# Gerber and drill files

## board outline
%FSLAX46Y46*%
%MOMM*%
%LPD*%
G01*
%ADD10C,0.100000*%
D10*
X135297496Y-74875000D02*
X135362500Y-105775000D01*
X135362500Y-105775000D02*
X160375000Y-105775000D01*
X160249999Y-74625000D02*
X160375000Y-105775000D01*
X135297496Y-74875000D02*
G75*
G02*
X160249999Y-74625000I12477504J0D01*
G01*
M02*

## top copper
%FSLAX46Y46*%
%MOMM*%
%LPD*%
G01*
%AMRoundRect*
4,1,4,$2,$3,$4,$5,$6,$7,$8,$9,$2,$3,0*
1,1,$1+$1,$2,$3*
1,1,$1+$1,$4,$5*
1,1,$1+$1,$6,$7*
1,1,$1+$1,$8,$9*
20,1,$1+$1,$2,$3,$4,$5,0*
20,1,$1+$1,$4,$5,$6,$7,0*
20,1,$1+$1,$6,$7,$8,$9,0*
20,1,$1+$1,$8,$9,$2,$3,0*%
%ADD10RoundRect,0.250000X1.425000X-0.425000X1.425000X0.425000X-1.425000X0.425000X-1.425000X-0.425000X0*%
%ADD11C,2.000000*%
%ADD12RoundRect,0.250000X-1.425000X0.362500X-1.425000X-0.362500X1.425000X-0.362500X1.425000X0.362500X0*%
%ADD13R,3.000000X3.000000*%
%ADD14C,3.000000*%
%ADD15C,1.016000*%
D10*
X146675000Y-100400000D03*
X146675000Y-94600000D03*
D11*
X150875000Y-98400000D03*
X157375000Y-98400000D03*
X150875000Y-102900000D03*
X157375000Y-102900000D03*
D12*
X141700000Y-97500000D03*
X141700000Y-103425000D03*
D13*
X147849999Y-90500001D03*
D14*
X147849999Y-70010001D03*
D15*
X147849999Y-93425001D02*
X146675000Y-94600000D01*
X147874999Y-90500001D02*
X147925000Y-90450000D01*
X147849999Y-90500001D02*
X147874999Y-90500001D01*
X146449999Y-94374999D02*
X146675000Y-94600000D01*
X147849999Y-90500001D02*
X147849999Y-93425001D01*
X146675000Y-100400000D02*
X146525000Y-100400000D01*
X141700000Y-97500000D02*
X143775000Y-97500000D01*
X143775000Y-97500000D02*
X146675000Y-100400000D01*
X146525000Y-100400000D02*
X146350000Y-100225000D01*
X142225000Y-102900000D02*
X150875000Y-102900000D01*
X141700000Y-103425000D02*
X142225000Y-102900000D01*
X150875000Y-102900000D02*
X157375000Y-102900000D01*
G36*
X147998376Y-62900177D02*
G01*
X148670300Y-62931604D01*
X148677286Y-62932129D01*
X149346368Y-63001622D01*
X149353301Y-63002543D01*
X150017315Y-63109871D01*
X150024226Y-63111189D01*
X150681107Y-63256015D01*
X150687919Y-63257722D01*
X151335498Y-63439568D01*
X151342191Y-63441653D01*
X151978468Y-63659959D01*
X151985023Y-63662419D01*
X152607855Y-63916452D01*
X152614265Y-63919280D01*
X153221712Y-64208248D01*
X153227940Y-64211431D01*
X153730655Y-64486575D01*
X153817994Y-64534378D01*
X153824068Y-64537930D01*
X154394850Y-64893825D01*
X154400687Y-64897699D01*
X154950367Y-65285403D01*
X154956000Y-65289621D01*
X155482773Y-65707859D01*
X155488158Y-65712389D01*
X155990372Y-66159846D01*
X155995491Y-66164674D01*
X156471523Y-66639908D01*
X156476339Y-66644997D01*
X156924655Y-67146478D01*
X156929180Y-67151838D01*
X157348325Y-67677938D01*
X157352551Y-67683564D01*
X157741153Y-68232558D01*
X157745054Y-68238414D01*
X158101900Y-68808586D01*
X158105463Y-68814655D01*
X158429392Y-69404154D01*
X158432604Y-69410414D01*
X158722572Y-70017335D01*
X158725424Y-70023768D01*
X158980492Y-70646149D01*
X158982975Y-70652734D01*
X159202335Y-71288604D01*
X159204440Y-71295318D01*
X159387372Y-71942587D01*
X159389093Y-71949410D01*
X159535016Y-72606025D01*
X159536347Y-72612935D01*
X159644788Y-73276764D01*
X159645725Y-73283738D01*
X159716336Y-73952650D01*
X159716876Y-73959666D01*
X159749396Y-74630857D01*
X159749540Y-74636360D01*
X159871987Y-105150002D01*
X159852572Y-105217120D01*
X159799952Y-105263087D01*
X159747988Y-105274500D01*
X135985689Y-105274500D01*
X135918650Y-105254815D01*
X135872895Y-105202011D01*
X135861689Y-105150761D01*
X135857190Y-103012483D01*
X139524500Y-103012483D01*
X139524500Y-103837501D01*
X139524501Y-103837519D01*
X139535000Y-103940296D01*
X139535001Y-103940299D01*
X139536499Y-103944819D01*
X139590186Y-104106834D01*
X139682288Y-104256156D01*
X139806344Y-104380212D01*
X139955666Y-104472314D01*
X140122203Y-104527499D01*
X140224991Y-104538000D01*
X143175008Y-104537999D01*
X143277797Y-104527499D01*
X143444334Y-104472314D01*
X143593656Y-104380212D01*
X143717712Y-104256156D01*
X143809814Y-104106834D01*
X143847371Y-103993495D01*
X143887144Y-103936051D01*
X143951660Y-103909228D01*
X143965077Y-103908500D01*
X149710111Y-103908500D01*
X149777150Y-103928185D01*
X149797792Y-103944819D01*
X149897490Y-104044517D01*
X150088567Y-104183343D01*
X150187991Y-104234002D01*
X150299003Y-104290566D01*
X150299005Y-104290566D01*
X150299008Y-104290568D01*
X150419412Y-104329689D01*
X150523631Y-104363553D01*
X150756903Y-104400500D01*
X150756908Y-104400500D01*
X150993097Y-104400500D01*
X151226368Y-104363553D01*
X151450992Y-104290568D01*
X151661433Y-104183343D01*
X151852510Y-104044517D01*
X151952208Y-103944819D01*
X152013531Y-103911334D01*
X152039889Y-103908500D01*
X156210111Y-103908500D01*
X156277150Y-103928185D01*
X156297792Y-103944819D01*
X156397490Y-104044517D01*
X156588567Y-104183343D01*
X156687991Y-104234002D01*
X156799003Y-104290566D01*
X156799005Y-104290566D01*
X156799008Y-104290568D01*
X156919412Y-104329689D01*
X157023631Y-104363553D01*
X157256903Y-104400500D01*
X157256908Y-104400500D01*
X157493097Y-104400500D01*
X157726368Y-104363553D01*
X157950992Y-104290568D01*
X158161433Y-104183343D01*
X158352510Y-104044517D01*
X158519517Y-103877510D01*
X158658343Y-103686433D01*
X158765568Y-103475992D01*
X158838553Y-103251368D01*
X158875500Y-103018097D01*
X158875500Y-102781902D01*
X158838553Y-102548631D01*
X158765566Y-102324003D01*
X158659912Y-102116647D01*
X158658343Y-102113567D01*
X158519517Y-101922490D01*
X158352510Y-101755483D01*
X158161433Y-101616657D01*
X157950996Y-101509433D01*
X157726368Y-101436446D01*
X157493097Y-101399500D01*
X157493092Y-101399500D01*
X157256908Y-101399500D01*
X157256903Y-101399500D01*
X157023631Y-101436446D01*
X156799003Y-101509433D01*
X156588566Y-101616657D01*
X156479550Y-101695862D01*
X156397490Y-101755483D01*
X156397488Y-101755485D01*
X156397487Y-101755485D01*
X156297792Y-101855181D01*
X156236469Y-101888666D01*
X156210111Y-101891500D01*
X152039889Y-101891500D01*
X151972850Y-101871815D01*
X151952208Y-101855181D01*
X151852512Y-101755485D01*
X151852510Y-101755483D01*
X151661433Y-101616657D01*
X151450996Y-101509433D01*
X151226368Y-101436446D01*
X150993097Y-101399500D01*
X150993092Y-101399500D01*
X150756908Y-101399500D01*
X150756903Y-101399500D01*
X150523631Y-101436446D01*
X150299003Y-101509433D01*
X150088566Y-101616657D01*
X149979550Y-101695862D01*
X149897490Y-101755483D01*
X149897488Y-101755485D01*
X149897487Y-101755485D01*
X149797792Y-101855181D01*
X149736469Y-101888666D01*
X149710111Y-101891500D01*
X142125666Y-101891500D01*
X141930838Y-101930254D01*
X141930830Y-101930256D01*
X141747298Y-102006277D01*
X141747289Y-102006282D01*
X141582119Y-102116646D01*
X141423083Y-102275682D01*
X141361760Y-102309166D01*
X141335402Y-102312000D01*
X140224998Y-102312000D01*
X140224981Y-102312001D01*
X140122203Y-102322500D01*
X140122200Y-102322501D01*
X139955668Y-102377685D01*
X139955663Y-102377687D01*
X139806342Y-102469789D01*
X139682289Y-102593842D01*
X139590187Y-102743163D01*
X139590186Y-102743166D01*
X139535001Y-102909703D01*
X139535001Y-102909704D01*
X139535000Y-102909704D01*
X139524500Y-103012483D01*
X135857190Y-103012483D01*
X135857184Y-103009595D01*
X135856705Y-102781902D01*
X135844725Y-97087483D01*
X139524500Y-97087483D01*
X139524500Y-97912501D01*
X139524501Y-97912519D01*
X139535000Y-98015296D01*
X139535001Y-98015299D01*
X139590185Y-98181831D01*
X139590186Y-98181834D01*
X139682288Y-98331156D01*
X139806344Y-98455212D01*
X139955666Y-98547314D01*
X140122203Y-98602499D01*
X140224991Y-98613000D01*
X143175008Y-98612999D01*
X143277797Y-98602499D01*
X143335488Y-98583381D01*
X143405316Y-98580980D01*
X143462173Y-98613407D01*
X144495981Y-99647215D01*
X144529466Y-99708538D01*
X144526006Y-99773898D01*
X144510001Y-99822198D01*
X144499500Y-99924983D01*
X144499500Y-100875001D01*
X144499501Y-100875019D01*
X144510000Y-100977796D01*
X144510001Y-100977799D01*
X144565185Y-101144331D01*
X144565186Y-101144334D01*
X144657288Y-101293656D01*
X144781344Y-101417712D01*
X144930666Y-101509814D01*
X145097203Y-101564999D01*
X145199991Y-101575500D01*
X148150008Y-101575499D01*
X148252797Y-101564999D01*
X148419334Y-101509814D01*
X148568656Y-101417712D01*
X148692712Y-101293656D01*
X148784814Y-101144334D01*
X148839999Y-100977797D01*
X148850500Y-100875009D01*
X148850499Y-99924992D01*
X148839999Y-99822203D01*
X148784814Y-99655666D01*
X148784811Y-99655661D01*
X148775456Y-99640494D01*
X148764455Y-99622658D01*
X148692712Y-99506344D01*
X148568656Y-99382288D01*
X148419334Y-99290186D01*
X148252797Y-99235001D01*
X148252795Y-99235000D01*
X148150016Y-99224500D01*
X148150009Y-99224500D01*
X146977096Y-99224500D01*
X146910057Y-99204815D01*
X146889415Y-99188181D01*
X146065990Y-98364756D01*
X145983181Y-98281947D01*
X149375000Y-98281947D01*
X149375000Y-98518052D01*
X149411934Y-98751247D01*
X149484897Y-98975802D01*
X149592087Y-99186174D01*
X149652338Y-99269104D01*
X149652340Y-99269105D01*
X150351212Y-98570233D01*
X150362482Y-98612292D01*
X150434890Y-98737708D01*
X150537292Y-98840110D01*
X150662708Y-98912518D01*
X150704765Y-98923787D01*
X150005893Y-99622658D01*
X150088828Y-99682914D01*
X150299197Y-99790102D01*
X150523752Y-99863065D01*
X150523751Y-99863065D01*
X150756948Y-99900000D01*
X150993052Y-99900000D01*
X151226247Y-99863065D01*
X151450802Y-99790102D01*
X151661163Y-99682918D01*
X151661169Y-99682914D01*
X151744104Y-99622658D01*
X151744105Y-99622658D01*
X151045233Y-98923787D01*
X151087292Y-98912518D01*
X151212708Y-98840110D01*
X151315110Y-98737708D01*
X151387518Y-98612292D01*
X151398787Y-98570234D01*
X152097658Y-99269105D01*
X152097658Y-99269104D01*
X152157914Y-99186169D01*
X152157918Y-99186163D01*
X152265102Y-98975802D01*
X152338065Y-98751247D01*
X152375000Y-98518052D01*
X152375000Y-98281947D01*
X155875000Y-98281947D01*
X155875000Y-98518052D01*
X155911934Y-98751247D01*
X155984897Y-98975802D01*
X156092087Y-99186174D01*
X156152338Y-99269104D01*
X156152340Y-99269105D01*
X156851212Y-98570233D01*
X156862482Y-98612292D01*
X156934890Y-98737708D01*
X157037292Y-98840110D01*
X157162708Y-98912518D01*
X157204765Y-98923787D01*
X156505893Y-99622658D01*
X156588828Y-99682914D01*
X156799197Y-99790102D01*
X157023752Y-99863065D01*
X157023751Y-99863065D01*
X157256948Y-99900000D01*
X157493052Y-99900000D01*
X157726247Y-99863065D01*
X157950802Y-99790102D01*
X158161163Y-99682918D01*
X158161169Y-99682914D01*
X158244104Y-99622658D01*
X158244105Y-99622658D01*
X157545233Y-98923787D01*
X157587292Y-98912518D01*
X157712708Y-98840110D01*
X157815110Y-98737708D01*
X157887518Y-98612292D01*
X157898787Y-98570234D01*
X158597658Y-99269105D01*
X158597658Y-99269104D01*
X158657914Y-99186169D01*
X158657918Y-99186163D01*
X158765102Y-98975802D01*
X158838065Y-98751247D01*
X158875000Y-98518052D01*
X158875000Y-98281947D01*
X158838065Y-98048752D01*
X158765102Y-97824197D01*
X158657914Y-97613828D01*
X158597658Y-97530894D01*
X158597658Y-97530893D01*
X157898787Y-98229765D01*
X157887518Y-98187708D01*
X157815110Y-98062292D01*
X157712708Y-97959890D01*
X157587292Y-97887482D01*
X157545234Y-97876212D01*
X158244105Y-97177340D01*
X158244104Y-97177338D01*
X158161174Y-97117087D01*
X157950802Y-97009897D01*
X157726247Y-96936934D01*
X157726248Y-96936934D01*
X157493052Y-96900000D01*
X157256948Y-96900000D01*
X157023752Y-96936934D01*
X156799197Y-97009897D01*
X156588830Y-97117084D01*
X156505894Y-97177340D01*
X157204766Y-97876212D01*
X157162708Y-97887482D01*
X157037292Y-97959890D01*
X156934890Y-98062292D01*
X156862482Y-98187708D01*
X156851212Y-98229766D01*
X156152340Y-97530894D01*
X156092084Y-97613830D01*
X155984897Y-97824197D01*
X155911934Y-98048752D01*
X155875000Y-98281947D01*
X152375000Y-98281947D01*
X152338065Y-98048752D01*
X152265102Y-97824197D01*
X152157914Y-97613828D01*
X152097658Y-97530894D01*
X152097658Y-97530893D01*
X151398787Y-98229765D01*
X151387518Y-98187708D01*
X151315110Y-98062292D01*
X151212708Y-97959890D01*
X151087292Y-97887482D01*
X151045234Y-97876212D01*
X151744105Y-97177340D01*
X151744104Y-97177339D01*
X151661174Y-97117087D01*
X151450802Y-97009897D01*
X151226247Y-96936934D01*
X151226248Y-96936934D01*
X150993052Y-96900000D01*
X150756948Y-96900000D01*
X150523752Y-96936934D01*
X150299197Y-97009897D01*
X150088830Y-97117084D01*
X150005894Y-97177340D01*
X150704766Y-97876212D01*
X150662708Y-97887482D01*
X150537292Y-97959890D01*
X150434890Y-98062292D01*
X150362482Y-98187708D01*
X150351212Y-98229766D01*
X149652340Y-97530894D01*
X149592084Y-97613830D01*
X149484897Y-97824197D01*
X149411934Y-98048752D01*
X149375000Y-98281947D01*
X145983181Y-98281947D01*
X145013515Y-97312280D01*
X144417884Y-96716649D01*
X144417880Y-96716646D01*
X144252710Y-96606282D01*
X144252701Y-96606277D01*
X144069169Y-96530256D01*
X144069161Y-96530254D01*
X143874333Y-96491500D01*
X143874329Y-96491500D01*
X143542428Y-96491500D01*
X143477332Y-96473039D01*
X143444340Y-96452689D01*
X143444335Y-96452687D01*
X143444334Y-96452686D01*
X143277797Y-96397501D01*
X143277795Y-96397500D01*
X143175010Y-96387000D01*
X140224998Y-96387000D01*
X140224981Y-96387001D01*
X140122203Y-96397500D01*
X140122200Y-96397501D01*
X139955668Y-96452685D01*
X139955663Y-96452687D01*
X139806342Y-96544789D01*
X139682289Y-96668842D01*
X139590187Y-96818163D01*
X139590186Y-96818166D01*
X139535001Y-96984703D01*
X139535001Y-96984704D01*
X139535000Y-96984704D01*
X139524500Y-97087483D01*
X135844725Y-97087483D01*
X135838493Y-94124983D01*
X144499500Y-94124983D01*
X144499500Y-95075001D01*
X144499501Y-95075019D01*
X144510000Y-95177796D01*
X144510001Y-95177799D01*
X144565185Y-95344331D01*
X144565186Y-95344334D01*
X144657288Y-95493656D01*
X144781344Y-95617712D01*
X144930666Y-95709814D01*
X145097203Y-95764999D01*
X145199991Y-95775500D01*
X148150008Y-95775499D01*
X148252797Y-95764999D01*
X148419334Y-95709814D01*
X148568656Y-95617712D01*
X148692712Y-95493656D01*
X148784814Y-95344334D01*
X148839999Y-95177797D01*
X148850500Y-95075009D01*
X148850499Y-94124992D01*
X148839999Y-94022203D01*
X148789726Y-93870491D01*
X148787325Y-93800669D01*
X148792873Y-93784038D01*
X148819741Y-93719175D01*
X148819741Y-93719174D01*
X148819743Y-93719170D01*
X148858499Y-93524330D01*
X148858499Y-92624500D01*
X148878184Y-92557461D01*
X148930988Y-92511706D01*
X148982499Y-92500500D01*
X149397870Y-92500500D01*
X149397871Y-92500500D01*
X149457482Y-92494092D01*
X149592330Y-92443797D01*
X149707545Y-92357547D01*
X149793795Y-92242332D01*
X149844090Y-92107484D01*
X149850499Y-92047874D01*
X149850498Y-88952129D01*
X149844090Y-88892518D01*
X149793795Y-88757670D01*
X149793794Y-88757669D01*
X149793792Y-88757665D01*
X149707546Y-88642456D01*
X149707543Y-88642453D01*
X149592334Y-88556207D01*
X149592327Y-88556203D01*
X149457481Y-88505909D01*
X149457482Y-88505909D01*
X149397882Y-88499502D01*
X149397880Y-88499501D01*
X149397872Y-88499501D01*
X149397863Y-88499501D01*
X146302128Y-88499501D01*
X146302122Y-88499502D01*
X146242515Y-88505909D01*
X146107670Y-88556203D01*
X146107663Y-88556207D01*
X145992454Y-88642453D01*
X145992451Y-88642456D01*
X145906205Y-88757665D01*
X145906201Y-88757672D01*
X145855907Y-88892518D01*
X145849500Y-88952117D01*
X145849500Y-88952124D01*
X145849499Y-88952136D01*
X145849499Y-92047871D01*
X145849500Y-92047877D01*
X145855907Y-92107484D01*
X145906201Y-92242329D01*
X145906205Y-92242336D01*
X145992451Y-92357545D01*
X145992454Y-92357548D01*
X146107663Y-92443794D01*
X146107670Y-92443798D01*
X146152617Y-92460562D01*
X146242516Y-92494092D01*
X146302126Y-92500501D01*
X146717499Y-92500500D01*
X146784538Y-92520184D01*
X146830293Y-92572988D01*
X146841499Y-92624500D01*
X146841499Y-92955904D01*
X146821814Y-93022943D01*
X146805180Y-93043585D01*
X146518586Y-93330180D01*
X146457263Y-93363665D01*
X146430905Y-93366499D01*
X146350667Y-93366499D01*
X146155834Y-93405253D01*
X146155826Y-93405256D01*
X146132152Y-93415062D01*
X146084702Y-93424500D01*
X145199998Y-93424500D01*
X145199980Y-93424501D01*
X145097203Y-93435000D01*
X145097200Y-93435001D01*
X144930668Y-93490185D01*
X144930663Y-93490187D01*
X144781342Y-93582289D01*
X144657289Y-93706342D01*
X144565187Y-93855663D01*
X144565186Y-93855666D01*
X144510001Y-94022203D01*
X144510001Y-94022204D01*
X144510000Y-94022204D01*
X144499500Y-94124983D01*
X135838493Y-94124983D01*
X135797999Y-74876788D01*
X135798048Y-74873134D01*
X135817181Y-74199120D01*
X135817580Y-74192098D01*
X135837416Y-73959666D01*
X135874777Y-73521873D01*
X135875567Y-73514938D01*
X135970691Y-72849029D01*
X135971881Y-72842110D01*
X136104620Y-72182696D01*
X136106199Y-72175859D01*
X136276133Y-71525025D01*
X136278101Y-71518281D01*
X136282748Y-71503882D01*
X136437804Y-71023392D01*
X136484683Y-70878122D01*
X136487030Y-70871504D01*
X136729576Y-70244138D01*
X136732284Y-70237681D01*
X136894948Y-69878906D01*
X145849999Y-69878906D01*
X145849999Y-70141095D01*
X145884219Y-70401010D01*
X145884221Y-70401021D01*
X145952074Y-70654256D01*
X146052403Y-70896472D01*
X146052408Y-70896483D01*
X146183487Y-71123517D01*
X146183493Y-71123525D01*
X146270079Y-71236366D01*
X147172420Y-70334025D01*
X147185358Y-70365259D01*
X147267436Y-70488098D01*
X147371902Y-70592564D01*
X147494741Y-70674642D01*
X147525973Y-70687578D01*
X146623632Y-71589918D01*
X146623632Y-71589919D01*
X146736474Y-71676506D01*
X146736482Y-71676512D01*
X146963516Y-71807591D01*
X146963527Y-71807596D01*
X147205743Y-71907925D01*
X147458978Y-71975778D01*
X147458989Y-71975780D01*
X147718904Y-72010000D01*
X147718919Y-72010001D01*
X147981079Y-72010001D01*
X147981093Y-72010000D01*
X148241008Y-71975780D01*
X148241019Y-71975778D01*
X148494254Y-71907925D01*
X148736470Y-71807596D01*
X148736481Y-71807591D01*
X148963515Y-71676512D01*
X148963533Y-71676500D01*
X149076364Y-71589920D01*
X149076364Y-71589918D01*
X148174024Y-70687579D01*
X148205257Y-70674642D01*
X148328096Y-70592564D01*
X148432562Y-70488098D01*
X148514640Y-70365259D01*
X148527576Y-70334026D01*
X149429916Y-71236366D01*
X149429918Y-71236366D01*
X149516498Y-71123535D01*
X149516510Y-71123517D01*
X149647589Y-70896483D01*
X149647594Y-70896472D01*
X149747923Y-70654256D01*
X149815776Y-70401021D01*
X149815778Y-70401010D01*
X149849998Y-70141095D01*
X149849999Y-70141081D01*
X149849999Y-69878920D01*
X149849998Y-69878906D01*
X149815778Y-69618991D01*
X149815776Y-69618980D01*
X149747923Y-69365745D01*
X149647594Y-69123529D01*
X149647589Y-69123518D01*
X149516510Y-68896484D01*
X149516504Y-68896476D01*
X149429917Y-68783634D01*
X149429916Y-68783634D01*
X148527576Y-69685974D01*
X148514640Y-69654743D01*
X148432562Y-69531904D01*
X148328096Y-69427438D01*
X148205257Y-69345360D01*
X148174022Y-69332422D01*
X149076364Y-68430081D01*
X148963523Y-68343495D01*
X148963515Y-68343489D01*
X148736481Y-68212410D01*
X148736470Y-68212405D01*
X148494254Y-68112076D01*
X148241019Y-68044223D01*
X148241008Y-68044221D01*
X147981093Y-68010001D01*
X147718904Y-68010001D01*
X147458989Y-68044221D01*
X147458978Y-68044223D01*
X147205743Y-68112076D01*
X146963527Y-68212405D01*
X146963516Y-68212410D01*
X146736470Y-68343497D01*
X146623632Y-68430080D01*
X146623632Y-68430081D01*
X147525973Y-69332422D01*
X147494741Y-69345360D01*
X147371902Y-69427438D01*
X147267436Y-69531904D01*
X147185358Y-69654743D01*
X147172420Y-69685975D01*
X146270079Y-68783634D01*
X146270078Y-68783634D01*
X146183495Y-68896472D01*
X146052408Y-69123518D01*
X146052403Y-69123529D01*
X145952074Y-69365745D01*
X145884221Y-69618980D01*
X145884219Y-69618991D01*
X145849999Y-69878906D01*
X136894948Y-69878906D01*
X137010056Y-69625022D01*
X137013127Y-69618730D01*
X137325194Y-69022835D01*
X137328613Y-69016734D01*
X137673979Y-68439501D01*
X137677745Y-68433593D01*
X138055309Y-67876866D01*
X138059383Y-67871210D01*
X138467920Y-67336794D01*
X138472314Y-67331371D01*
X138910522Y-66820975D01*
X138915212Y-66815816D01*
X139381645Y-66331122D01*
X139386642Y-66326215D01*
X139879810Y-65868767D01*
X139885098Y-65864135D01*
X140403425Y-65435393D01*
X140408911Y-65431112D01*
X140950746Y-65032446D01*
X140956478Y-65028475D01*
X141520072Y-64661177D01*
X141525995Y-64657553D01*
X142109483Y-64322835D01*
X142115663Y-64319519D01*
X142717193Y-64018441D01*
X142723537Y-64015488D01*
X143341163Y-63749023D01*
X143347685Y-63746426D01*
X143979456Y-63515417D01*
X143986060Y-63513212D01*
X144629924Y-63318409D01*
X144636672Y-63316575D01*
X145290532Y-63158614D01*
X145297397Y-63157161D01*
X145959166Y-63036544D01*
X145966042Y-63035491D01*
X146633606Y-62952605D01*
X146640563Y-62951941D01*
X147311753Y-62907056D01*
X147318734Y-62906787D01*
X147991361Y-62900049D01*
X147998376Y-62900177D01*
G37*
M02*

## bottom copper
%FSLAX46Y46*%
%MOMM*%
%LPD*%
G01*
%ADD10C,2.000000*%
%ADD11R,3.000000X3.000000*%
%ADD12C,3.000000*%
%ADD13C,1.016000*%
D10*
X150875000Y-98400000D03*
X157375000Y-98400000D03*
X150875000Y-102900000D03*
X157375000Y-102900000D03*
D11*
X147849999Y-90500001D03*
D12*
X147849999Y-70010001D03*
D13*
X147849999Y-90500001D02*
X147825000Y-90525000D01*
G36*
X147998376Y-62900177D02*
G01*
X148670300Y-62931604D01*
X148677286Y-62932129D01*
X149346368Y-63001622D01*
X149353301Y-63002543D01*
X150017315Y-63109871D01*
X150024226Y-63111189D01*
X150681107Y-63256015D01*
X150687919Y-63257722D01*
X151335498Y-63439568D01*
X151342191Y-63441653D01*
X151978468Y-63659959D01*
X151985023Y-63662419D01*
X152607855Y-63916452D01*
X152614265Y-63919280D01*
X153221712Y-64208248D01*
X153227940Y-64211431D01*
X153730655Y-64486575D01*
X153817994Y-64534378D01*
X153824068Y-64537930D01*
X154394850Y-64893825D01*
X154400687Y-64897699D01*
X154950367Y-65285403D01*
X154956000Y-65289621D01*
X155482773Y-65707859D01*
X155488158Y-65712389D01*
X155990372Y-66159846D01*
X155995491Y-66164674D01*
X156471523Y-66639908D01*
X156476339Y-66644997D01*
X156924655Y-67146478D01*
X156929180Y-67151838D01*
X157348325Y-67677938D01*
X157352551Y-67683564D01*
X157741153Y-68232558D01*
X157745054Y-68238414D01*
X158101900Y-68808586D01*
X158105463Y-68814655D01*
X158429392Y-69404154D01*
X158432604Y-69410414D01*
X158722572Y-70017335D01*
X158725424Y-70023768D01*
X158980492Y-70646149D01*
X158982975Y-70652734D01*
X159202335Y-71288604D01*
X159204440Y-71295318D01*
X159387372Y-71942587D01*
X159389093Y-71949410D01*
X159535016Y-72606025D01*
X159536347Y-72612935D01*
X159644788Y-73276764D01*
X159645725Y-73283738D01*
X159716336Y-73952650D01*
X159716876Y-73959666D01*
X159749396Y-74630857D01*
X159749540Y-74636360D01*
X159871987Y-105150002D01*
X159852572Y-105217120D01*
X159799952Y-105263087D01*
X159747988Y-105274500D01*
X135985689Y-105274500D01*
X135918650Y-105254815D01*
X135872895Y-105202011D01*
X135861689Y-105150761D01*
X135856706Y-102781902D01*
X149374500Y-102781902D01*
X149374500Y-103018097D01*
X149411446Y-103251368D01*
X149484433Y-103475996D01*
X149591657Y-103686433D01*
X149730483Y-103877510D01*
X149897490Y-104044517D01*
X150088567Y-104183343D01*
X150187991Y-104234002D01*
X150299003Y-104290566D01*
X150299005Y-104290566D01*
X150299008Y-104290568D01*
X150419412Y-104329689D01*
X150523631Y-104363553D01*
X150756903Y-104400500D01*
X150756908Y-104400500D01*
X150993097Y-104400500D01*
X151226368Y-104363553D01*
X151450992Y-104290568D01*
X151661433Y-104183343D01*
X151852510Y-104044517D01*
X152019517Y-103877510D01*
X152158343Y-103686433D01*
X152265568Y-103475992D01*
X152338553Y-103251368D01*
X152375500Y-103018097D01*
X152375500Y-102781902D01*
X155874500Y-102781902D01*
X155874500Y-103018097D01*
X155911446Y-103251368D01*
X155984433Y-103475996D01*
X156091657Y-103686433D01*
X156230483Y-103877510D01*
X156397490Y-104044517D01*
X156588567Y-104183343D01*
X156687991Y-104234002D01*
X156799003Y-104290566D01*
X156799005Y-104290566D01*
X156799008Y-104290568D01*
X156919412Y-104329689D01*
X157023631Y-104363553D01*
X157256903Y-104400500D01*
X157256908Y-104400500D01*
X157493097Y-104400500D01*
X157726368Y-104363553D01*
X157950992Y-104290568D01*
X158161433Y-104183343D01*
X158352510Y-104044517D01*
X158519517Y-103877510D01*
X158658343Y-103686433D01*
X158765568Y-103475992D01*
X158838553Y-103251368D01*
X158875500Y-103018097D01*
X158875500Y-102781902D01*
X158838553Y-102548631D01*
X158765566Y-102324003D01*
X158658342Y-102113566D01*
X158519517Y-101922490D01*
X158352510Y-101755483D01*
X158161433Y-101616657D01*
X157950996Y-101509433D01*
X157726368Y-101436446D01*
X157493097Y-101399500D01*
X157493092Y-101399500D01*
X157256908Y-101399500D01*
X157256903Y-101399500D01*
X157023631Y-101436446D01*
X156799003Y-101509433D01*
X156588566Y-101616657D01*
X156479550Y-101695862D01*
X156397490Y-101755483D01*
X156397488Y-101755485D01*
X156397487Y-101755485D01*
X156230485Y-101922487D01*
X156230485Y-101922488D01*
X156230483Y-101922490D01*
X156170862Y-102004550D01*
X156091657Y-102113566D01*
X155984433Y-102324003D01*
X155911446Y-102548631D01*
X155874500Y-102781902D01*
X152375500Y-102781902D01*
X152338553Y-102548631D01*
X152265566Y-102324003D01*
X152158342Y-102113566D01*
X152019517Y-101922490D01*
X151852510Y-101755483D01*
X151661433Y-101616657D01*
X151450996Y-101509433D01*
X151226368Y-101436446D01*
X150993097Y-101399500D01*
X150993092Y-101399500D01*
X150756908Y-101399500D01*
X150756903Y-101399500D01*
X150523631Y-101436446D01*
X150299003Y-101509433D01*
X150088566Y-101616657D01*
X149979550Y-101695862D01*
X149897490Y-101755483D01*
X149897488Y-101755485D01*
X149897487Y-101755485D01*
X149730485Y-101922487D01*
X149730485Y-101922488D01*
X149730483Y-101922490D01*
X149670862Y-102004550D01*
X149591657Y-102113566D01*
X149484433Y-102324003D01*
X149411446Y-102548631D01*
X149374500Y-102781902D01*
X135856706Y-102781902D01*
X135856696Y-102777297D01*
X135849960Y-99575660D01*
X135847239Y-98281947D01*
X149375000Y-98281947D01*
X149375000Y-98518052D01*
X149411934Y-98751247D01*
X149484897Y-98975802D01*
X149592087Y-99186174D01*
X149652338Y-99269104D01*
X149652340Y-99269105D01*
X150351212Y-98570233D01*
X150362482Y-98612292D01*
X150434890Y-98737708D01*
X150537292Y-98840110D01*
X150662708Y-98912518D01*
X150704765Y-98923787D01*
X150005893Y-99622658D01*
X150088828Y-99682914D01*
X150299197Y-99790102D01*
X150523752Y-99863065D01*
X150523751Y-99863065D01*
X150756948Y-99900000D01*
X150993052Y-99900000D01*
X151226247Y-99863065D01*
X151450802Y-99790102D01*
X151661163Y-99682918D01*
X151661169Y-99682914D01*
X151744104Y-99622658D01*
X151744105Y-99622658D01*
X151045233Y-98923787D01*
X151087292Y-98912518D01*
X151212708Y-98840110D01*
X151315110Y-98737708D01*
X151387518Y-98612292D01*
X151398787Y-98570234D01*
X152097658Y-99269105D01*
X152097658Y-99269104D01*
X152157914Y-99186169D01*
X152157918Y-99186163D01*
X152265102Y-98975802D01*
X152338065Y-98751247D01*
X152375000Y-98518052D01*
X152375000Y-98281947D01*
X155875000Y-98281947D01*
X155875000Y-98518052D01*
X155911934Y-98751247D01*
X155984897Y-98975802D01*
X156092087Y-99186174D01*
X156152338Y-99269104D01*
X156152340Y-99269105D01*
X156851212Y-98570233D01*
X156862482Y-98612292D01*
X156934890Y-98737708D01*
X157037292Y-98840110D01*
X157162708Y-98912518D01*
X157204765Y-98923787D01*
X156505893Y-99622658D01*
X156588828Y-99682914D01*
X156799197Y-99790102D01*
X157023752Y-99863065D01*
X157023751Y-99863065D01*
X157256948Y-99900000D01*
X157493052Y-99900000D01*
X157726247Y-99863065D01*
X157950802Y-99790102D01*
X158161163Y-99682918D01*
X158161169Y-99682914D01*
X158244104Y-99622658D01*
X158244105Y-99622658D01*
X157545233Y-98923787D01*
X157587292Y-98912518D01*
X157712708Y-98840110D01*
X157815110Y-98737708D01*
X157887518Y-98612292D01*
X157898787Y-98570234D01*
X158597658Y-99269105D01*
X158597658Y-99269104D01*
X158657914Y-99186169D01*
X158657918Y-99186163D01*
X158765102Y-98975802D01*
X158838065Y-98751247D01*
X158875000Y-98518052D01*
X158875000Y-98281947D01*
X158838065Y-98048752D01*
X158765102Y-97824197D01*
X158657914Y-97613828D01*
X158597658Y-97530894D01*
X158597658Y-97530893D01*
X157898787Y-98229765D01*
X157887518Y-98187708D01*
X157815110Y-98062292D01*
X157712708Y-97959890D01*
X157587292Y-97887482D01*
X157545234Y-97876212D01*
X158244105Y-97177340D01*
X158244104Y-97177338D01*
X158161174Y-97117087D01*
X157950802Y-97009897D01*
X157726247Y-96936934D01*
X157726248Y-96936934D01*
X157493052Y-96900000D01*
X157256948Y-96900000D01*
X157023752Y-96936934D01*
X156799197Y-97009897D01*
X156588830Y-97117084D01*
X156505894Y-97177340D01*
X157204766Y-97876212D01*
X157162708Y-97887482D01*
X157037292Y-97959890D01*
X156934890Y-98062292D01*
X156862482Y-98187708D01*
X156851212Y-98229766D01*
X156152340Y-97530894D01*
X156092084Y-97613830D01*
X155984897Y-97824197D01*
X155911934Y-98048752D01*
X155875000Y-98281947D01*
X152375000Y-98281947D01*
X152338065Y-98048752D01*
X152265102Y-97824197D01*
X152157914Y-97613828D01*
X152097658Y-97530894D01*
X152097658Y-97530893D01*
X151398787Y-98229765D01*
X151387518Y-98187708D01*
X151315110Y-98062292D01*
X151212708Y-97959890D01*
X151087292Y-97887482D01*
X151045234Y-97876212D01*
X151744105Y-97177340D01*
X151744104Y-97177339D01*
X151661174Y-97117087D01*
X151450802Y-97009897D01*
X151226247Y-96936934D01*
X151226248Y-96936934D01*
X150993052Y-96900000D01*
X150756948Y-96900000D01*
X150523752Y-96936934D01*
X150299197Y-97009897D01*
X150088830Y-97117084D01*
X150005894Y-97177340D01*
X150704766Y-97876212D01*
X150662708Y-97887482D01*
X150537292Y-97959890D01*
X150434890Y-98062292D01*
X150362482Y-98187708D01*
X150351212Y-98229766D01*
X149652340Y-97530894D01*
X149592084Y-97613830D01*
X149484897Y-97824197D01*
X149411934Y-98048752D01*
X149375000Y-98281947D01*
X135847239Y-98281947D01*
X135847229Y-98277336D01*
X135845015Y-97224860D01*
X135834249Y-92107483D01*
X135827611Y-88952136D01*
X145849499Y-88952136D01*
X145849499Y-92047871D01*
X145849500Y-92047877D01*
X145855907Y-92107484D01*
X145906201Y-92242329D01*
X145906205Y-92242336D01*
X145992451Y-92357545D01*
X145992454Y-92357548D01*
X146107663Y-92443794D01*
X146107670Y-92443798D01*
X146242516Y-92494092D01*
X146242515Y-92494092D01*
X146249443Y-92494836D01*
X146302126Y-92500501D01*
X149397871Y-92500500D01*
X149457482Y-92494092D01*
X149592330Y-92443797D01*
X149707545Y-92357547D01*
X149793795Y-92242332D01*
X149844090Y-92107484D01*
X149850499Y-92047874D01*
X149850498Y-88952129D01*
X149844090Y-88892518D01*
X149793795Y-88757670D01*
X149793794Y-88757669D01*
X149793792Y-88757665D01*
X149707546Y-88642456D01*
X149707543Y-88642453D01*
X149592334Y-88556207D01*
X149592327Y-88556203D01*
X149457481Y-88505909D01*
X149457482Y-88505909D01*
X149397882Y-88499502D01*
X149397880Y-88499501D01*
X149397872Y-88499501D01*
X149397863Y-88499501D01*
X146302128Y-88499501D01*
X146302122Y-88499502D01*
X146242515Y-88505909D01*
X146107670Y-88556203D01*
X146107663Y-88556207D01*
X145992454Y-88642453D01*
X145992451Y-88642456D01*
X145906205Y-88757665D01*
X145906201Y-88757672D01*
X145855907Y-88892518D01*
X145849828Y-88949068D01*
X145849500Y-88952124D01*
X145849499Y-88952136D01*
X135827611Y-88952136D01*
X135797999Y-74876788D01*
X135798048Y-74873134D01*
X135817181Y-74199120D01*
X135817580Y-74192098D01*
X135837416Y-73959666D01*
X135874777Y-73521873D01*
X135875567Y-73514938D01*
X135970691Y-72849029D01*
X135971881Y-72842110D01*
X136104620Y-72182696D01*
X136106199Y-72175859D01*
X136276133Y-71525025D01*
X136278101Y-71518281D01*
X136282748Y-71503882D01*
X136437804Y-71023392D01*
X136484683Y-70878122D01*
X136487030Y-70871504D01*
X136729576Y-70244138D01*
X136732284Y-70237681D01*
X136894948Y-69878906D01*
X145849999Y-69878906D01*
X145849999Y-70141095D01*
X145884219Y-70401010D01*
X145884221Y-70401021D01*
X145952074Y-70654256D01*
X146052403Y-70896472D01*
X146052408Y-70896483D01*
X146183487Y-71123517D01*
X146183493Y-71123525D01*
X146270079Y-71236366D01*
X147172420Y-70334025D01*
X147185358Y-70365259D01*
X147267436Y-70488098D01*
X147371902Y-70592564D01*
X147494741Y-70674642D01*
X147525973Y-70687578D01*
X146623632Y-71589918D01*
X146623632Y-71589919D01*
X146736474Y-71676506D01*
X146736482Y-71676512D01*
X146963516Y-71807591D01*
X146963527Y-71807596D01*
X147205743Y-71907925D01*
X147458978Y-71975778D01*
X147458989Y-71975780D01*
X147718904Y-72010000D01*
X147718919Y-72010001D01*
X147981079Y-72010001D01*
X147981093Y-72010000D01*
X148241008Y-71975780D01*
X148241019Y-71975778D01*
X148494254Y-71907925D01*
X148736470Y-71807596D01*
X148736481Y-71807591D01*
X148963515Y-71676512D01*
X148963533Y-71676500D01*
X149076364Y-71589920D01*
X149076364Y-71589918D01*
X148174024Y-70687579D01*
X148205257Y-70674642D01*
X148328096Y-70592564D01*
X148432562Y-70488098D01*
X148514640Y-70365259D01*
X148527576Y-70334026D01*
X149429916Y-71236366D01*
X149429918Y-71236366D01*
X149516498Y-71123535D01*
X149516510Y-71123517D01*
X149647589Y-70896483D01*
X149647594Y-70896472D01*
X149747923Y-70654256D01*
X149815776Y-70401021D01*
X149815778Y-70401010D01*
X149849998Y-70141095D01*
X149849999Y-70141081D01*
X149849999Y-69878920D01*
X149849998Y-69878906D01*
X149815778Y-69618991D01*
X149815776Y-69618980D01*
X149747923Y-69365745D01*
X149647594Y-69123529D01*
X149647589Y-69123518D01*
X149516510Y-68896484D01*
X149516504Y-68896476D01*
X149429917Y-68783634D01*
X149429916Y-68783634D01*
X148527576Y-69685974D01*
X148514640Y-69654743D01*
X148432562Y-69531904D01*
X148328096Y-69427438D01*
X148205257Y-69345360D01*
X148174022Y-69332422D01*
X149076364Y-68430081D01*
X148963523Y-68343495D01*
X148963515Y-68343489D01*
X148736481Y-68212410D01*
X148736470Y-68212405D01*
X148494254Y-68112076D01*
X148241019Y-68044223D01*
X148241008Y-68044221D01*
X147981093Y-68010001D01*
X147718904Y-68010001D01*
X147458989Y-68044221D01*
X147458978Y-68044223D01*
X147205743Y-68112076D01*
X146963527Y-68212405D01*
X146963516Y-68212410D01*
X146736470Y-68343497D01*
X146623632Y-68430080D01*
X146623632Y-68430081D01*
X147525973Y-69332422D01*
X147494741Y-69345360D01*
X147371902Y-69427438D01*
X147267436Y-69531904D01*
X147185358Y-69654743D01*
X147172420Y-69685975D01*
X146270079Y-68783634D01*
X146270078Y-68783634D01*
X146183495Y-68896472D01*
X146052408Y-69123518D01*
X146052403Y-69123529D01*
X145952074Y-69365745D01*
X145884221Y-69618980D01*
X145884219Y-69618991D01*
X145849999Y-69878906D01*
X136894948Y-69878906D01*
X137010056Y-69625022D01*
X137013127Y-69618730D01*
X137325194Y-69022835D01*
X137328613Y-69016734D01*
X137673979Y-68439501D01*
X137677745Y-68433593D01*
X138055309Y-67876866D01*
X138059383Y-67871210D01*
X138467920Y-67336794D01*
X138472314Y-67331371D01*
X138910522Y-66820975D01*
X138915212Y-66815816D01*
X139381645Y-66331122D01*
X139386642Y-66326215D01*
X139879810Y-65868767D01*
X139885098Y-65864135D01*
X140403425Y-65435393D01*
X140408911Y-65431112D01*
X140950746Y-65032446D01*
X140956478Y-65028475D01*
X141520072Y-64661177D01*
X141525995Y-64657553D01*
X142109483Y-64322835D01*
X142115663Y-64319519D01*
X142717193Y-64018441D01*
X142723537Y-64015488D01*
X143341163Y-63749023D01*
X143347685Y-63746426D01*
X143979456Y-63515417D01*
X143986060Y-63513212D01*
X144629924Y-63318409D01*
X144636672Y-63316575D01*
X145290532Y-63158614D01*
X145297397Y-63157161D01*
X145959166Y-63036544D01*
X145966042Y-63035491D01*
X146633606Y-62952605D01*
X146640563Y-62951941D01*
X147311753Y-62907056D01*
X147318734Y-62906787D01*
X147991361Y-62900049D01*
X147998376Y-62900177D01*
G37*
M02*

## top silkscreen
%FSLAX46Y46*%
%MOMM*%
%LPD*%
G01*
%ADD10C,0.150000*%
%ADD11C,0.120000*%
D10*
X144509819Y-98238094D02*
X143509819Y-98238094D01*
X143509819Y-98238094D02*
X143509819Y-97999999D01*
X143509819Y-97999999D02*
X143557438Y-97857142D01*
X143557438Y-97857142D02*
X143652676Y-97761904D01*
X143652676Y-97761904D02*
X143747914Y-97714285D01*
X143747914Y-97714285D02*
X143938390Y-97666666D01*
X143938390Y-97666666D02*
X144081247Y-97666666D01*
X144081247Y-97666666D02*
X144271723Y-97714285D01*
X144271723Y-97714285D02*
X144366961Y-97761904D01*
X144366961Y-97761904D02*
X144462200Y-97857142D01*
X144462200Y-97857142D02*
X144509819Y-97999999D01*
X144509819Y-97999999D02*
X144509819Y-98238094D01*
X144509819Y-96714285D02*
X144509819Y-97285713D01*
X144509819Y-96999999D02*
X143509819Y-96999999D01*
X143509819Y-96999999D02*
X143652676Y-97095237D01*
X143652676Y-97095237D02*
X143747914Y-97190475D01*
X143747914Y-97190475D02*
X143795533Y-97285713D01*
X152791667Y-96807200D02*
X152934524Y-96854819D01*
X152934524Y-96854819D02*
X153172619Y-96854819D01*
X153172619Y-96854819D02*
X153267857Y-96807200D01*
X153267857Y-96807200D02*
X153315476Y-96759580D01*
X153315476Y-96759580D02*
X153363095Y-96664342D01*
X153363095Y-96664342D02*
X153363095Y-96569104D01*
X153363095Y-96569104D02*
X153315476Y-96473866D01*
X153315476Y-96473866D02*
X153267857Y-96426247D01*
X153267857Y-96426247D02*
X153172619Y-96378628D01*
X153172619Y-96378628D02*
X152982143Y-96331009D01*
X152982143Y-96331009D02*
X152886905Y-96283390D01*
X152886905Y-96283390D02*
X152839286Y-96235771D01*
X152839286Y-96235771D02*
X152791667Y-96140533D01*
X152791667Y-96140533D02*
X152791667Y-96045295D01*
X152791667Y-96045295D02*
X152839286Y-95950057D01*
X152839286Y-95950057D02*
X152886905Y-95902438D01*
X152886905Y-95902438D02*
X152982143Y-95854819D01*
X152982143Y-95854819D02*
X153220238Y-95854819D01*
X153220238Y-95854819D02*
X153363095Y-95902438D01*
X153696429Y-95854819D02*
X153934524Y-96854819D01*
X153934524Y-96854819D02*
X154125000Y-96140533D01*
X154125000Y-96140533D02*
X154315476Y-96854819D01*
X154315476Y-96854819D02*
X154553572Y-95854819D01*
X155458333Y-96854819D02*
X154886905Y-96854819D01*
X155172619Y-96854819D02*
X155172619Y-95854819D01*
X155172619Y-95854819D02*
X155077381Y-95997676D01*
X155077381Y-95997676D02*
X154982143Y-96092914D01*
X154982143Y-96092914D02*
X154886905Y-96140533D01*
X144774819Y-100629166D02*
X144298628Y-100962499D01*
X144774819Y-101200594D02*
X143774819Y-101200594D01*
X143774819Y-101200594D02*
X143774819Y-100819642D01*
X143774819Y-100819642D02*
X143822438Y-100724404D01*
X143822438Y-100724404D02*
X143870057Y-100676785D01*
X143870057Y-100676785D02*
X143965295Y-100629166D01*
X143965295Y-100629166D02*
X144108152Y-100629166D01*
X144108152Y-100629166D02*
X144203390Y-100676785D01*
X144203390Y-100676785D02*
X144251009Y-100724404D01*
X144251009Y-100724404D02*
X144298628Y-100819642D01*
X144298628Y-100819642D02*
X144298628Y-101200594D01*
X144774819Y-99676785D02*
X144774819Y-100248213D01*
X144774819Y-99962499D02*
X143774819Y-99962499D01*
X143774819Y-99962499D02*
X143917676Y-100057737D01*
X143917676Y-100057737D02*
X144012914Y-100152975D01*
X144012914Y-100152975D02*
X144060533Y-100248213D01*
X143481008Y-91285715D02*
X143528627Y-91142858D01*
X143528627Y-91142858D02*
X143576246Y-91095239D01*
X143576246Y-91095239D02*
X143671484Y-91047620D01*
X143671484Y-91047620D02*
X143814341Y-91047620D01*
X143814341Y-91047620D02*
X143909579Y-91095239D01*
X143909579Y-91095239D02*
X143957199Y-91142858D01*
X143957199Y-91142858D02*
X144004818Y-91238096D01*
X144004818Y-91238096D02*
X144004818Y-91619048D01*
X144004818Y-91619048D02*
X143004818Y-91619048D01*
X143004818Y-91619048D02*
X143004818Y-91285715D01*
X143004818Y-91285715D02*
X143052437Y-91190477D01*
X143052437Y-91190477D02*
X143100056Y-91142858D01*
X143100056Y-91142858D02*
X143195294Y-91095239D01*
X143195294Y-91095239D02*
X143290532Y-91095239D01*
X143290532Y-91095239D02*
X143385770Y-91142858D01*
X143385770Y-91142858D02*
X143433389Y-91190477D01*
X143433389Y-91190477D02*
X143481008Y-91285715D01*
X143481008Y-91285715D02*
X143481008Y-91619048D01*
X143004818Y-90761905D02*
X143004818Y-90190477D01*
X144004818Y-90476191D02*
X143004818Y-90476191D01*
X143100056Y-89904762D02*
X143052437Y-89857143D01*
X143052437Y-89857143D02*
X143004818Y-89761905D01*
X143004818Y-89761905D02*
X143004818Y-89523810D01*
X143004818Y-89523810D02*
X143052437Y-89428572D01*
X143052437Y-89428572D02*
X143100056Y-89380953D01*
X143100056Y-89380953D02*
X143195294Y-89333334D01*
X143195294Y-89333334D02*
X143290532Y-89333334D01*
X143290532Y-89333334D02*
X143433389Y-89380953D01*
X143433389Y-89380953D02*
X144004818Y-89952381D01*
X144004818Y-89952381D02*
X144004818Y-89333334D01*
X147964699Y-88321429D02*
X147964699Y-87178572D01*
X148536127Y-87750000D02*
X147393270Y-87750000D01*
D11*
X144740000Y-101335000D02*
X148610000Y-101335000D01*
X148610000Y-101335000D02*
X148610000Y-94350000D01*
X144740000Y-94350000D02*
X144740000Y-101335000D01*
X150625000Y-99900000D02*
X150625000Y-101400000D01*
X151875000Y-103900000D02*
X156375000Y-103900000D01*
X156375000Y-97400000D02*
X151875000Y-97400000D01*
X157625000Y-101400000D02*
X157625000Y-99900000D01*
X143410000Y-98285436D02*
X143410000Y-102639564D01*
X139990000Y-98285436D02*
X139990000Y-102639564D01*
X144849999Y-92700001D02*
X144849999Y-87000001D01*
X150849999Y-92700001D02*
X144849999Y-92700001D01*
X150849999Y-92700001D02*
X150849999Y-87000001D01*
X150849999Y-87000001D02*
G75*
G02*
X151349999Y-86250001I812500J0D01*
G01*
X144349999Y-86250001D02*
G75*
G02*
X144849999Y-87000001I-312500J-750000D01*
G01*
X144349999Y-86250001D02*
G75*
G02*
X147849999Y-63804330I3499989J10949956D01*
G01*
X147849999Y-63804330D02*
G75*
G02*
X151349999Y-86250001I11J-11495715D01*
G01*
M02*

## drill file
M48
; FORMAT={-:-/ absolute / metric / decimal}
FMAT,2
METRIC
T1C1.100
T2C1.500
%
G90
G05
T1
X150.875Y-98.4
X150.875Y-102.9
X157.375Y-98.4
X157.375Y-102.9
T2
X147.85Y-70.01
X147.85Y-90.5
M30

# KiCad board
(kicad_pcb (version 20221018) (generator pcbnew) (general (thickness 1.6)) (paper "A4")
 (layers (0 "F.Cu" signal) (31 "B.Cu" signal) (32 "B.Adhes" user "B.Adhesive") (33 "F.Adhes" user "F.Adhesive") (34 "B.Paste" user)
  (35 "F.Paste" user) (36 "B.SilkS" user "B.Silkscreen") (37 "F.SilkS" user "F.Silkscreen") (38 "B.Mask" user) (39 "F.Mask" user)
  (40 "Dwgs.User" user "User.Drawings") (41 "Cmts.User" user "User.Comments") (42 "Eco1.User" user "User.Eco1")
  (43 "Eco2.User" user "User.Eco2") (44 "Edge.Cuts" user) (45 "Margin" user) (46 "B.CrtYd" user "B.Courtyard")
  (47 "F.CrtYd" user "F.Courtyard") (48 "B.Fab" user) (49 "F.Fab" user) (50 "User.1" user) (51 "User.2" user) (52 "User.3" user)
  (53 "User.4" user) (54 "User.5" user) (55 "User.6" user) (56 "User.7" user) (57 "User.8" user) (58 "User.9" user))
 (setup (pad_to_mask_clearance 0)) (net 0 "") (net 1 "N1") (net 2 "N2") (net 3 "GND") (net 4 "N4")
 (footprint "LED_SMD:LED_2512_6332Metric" (layer "F.Cu") (at 146.675 97.5 90)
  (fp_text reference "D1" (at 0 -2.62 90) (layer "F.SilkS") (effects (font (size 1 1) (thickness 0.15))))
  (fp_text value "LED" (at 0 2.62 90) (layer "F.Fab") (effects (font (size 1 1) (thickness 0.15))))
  (fp_line (start -3.835 -1.935) (end -3.835 1.935) (stroke (width 0.12) (type solid)) (layer "F.SilkS"))
  (fp_line (start -3.835 1.935) (end 3.15 1.935) (stroke (width 0.12) (type solid)) (layer "F.SilkS"))
  (fp_line (start 3.15 -1.935) (end -3.835 -1.935) (stroke (width 0.12) (type solid)) (layer "F.SilkS"))
  (pad "1" smd roundrect (at -2.9 0 90) (size 1.35 3.35) (layers "F.Cu" "F.Paste" "F.Mask") (roundrect_rratio 0.185185) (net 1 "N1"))
  (pad "2" smd roundrect (at 2.9 0 90) (size 1.35 3.35) (layers "F.Cu" "F.Paste" "F.Mask") (roundrect_rratio 0.185185) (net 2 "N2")))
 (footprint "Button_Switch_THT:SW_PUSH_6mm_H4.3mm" (layer "F.Cu") (at 150.875 98.4)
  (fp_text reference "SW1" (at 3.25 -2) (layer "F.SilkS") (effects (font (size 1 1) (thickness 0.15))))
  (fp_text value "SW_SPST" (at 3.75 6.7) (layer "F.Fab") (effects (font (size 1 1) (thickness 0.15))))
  (fp_line (start -0.25 1.5) (end -0.25 3) (stroke (width 0.12) (type solid)) (layer "F.SilkS"))
  (fp_line (start 1 5.5) (end 5.5 5.5) (stroke (width 0.12) (type solid)) (layer "F.SilkS"))
  (fp_line (start 5.5 -1) (end 1 -1) (stroke (width 0.12) (type solid)) (layer "F.SilkS"))
  (fp_line (start 6.75 3) (end 6.75 1.5) (stroke (width 0.12) (type solid)) (layer "F.SilkS"))
  (pad "1" thru_hole circle (at 0 0 90) (size 2 2) (drill 1.1) (layers "*.Cu" "*.Mask") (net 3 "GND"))
  (pad "1" thru_hole circle (at 6.5 0 90) (size 2 2) (drill 1.1) (layers "*.Cu" "*.Mask") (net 3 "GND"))
  (pad "2" thru_hole circle (at 0 4.5 90) (size 2 2) (drill 1.1) (layers "*.Cu" "*.Mask") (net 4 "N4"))
  (pad "2" thru_hole circle (at 6.5 4.5 90) (size 2 2) (drill 1.1) (layers "*.Cu" "*.Mask") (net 4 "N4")))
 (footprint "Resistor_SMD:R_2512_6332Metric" (layer "F.Cu") (at 141.7 100.4625 -90)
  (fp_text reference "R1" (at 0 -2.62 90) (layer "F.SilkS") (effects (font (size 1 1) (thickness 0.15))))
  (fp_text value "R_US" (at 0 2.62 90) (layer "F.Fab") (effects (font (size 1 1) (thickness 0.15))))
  (fp_line (start -2.177064 -1.71) (end 2.177064 -1.71) (stroke (width 0.12) (type solid)) (layer "F.SilkS"))
  (fp_line (start -2.177064 1.71) (end 2.177064 1.71) (stroke (width 0.12) (type solid)) (layer "F.SilkS"))
  (pad "1" smd roundrect (at -2.9625 0 270) (size 1.225 3.35) (layers "F.Cu" "F.Paste" "F.Mask") (roundrect_rratio 0.204082) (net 1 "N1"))
  (pad "2" smd roundrect (at 2.9625 0 270) (size 1.225 3.35) (layers "F.Cu" "F.Paste" "F.Mask") (roundrect_rratio 0.204082) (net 4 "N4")))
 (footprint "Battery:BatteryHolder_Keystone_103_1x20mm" (layer "F.Cu") (at 147.849999 90.500001 90)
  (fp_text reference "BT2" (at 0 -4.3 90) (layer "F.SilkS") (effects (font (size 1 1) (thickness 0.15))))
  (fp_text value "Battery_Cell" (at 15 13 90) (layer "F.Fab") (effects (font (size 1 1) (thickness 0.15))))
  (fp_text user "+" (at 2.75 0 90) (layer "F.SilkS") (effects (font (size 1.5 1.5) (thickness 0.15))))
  (fp_line (start -2.2 -3) (end 3.5 -3) (stroke (width 0.12) (type solid)) (layer "F.SilkS"))
  (fp_line (start -2.2 3) (end -2.2 -3) (stroke (width 0.12) (type solid)) (layer "F.SilkS"))
  (fp_line (start -2.2 3) (end 3.5 3) (stroke (width 0.12) (type solid)) (layer "F.SilkS"))
  (fp_arc (start 3.5 3) (mid 3.950694 3.136459) (end 4.25 3.5) (stroke (width 0.12) (type solid)) (layer "F.SilkS"))
  (fp_arc (start 4.25 -3.5) (mid 3.950694 -3.136459) (end 3.5 -3) (stroke (width 0.12) (type solid)) (layer "F.SilkS"))
  (fp_arc (start 4.25 -3.5) (mid 16.971103 -11.358466) (end 26.695671 0) (stroke (width 0.12) (type solid)) (layer "F.SilkS"))
  (fp_arc (start 26.695671 0) (mid 16.971103 11.358466) (end 4.25 3.5) (stroke (width 0.12) (type solid)) (layer "F.SilkS"))
  (pad "1" thru_hole rect (at 0 0 90) (size 3 3) (drill 1.5) (layers "*.Cu" "*.Mask") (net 2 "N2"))
  (pad "2" thru_hole circle (at 20.49 0 90) (size 3 3) (drill 1.5) (layers "*.Cu" "*.Mask") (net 3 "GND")))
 (gr_line (start 135.297496 74.875) (end 135.3625 105.775) (stroke (width 0.1) (type default)) (layer "Edge.Cuts"))
 (gr_line (start 135.3625 105.775) (end 160.375 105.775) (stroke (width 0.1) (type default)) (layer "Edge.Cuts"))
 (gr_line (start 160.249999 74.625) (end 160.375 105.775) (stroke (width 0.1) (type default)) (layer "Edge.Cuts"))
 (gr_arc (start 135.297496 74.875) (mid 147.649994 62.398122) (end 160.249999 74.625) (stroke (width 0.1) (type default))
  (layer "Edge.Cuts"))
 (segment (start 147.849999 93.425001) (end 146.675 94.6) (width 1.016) (layer "F.Cu") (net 2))
 (segment (start 147.874999 90.500001) (end 147.925 90.45) (width 1.016) (layer "F.Cu") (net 2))
 (segment (start 147.849999 90.500001) (end 147.874999 90.500001) (width 1.016) (layer "F.Cu") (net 2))
 (segment (start 146.449999 94.374999) (end 146.675 94.6) (width 1.016) (layer "F.Cu") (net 2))
 (segment (start 147.849999 90.500001) (end 147.849999 93.425001) (width 1.016) (layer "F.Cu") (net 2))
 (segment (start 147.849999 90.500001) (end 147.825 90.525) (width 1.016) (layer "B.Cu") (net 2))
 (segment (start 146.675 100.4) (end 146.525 100.4) (width 1.016) (layer "F.Cu") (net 1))
 (segment (start 141.7 97.5) (end 143.775 97.5) (width 1.016) (layer "F.Cu") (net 1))
 (segment (start 143.775 97.5) (end 146.675 100.4) (width 1.016) (layer "F.Cu") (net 1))
 (segment (start 146.525 100.4) (end 146.35 100.225) (width 1.016) (layer "F.Cu") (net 1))
 (segment (start 142.225 102.9) (end 150.875 102.9) (width 1.016) (layer "F.Cu") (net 4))
 (segment (start 141.7 103.425) (end 142.225 102.9) (width 1.016) (layer "F.Cu") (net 4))
 (segment (start 150.875 102.9) (end 157.375 102.9) (width 1.016) (layer "F.Cu") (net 4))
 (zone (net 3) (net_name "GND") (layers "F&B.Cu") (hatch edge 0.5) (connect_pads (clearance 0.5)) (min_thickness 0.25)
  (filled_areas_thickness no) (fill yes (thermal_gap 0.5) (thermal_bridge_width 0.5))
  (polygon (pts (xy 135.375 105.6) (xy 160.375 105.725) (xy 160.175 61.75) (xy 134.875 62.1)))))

